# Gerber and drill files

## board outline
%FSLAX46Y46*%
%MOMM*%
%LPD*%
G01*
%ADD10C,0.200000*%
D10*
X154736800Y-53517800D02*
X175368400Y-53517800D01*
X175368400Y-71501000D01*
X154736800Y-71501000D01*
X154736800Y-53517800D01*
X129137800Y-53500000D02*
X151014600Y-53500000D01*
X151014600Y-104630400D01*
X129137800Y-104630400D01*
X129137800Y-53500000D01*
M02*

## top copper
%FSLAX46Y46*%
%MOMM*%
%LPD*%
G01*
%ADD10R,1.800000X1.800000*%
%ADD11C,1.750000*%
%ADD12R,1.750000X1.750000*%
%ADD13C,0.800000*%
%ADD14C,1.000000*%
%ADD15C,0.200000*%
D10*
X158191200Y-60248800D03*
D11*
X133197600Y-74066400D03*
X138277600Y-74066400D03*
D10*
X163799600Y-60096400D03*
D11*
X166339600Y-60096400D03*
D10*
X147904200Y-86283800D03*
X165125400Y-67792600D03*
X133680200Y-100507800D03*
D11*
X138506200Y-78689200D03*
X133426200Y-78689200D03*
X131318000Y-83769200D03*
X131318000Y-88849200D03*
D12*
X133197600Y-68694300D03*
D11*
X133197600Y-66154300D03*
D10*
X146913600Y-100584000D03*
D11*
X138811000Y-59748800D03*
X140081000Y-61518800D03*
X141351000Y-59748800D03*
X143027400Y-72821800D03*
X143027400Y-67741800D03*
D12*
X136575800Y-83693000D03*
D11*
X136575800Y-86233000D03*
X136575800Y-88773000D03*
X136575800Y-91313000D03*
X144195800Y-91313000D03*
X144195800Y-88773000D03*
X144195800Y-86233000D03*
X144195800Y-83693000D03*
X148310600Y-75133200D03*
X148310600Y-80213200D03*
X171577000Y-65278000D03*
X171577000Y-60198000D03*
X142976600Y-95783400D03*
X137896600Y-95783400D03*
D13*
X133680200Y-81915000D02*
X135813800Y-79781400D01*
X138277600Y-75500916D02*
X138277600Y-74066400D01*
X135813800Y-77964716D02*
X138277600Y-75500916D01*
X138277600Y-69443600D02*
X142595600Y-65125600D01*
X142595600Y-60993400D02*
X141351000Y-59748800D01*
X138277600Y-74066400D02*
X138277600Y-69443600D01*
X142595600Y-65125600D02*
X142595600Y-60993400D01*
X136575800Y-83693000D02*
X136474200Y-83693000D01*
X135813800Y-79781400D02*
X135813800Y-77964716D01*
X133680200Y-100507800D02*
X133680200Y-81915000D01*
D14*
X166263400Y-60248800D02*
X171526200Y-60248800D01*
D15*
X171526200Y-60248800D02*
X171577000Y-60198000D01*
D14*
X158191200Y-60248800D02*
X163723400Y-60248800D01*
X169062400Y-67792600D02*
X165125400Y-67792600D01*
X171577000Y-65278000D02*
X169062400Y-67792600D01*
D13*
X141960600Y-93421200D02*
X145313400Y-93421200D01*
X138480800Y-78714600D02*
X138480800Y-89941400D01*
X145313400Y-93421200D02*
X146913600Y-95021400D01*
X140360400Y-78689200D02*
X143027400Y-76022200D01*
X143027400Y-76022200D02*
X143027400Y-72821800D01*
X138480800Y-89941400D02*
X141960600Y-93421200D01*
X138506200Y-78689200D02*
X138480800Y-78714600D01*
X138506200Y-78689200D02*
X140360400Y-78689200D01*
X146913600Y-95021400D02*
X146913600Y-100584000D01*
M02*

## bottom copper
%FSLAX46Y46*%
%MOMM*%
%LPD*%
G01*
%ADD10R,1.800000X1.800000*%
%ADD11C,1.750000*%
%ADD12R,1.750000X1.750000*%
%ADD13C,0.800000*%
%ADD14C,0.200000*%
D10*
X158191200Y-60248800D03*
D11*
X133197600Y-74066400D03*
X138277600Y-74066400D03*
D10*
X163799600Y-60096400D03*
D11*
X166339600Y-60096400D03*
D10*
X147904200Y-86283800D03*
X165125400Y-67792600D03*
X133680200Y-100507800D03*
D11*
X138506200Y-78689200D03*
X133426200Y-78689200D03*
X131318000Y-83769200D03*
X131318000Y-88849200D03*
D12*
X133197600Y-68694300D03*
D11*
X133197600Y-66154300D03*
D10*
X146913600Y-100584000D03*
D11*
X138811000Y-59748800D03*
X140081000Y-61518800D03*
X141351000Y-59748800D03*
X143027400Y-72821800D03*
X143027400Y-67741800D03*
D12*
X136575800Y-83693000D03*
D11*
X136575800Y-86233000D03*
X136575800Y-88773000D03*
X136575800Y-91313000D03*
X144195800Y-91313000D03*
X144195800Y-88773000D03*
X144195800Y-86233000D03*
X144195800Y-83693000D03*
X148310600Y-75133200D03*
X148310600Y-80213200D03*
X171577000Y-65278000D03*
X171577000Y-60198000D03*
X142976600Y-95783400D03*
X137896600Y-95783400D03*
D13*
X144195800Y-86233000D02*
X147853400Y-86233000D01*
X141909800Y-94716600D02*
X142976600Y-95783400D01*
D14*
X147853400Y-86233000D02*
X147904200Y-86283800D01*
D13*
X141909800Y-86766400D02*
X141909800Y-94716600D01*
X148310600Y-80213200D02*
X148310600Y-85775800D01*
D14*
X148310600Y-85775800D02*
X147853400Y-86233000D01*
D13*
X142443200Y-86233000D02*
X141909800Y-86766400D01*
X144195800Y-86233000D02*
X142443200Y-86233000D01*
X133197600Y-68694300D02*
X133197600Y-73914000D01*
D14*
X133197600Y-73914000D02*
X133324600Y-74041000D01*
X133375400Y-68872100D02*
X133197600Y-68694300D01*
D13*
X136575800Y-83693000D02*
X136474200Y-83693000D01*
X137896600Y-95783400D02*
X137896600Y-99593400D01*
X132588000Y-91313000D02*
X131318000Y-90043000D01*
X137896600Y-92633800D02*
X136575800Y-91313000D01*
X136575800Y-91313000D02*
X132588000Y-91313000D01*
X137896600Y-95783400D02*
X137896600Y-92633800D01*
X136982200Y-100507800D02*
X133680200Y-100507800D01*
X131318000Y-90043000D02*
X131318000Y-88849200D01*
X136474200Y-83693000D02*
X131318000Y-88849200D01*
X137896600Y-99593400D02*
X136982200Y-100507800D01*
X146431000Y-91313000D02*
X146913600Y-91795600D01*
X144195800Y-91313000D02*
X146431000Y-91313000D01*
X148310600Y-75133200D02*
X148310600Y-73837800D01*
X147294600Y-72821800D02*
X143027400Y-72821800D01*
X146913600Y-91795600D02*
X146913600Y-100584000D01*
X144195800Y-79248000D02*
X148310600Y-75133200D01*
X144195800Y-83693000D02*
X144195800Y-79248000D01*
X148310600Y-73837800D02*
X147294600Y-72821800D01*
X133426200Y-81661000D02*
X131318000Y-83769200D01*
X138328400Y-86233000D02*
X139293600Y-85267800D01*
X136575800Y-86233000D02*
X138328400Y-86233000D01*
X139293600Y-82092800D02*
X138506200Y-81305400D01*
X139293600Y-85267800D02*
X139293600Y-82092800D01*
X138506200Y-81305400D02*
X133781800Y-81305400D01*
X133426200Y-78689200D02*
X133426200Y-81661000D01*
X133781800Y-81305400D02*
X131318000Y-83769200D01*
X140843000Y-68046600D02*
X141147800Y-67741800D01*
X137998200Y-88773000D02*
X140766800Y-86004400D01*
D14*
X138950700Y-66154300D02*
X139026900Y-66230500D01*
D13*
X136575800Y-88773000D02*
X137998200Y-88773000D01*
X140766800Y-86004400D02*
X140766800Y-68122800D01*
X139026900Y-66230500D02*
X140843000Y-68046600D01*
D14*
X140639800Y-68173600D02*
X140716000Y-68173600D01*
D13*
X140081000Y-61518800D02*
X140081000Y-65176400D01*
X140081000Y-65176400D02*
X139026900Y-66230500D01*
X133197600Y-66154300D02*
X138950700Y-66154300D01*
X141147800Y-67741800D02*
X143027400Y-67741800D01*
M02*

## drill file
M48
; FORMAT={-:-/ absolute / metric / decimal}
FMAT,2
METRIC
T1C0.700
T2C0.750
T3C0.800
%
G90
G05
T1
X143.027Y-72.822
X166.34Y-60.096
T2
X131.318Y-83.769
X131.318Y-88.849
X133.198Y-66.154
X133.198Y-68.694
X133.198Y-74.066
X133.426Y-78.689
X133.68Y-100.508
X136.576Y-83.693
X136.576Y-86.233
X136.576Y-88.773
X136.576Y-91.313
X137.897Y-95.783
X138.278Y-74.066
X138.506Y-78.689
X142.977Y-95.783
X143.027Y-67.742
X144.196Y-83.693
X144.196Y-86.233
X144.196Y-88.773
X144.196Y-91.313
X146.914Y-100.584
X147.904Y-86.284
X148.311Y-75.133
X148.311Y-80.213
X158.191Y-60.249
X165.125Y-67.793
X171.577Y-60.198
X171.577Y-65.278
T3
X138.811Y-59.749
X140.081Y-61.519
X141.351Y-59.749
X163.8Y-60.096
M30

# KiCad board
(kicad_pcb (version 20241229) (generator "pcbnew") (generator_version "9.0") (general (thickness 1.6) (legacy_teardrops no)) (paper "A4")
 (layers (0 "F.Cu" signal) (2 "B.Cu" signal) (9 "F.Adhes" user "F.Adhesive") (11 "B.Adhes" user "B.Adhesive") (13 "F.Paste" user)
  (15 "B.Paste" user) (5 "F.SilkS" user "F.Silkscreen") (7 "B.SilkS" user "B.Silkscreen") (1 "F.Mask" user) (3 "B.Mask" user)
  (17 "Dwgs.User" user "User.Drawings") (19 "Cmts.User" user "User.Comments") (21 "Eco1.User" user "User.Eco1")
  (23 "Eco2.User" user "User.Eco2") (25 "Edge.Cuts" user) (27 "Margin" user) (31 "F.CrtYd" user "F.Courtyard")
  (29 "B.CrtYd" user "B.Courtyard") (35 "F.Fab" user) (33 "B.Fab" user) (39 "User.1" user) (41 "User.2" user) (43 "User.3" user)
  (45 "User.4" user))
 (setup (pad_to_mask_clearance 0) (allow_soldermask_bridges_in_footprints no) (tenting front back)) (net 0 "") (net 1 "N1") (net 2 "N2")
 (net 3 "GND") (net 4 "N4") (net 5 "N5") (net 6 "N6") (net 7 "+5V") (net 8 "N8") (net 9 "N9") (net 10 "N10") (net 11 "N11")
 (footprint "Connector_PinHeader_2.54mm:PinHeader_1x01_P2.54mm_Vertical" (layer "F.Cu") (at 158.1912 60.2488)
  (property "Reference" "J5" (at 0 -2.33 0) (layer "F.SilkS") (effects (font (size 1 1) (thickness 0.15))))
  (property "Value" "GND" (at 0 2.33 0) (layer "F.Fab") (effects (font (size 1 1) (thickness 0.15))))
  (pad "1" thru_hole rect (at 0 0) (size 1.8 1.8) (drill 0.75) (layers "*.Cu" "*.Mask") (remove_unused_layers no) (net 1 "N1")))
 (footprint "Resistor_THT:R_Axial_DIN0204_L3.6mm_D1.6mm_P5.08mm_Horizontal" (layer "F.Cu") (at 133.1976 74.0664)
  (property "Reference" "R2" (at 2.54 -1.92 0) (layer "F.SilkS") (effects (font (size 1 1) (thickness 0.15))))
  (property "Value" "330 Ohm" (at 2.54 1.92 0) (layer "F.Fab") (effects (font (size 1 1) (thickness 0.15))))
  (pad "1" thru_hole circle (at 0 0) (size 1.75 1.75) (drill 0.75) (layers "*.Cu" "*.Mask") (remove_unused_layers no) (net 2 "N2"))
  (pad "2" thru_hole circle (at 5.08 0) (size 1.75 1.75) (drill 0.75) (layers "*.Cu" "*.Mask") (remove_unused_layers no) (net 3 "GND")))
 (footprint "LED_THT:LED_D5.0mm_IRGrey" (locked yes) (layer "F.Cu") (at 163.7996 60.0964)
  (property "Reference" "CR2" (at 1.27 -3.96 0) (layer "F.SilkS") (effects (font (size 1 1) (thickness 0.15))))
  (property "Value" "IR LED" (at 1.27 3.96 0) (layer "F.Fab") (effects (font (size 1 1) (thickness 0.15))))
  (pad "1" thru_hole rect (at 0 0) (size 1.8 1.8) (drill 0.8) (layers "*.Cu" "*.Mask") (remove_unused_layers no) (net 1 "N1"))
  (pad "2" thru_hole circle (at 2.54 0) (size 1.75 1.75) (drill 0.7) (layers "*.Cu" "*.Mask") (remove_unused_layers no) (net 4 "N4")))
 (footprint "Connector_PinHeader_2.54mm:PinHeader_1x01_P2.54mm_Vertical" (layer "F.Cu") (at 147.9042 86.2838)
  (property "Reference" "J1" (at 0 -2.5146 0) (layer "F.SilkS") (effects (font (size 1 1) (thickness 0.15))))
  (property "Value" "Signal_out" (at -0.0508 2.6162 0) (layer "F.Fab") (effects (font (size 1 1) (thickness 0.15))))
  (pad "1" thru_hole rect (at 0 0) (size 1.8 1.8) (drill 0.75) (layers "*.Cu" "*.Mask") (remove_unused_layers no) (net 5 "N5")))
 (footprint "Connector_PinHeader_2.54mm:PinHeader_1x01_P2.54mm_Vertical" (layer "F.Cu") (at 165.1254 67.7926)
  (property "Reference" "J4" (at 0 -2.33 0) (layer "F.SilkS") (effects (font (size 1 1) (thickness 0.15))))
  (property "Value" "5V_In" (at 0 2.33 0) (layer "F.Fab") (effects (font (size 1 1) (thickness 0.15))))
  (pad "1" thru_hole rect (at 0 0) (size 1.8 1.8) (drill 0.75) (layers "*.Cu" "*.Mask") (remove_unused_layers no) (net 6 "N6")))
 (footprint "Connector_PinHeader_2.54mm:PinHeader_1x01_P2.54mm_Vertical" (layer "F.Cu") (at 133.6802 100.5078)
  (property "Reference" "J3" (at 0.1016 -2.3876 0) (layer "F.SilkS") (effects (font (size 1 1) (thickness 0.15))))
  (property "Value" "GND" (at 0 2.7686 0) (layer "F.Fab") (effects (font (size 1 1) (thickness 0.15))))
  (pad "1" thru_hole rect (at 0 0) (size 1.8 1.8) (drill 0.75) (layers "*.Cu" "*.Mask") (remove_unused_layers no) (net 3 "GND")))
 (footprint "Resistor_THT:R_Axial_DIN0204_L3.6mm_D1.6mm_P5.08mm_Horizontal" (layer "F.Cu") (at 138.5062 78.6892 180)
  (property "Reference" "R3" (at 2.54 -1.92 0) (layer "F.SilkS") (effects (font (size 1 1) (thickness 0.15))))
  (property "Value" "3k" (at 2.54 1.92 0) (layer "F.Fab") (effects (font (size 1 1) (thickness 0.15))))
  (pad "1" thru_hole circle (at 0 0 180) (size 1.75 1.75) (drill 0.75) (layers "*.Cu" "*.Mask") (remove_unused_layers no) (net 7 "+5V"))
  (pad "2" thru_hole circle (at 5.08 0 180) (size 1.75 1.75) (drill 0.75) (layers "*.Cu" "*.Mask") (remove_unused_layers no) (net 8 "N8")))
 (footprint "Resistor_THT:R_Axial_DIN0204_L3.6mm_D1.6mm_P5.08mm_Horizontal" (layer "F.Cu") (at 131.318 83.7692 -90)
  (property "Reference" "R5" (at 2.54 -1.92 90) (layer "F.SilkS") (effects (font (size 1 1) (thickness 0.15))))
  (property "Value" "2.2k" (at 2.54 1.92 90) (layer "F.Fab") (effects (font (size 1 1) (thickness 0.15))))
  (pad "1" thru_hole circle (at 0 0 270) (size 1.75 1.75) (drill 0.75) (layers "*.Cu" "*.Mask") (remove_unused_layers no) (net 8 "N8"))
  (pad "2" thru_hole circle (at 5.08 0 270) (size 1.75 1.75) (drill 0.75) (layers "*.Cu" "*.Mask") (remove_unused_layers no) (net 3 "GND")))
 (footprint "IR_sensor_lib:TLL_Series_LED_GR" (layer "F.Cu") (at 133.1976 68.6943 90)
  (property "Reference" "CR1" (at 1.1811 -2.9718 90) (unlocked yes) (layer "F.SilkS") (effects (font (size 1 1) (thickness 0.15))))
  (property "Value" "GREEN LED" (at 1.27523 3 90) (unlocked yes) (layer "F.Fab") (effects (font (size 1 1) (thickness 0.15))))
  (pad "1" thru_hole rect (at 0 0 90) (size 1.75 1.75) (drill 0.75) (layers "*.Cu" "*.Mask") (remove_unused_layers no) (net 2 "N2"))
  (pad "2" thru_hole circle (at 2.54 0 90) (size 1.75 1.75) (drill 0.75) (layers "*.Cu" "*.Mask") (remove_unused_layers no) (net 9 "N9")))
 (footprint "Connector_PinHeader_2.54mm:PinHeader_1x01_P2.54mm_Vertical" (layer "F.Cu") (at 146.9136 100.584)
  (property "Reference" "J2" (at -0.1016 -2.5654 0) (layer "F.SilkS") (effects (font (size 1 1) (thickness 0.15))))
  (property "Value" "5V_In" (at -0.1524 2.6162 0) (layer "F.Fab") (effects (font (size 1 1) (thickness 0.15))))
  (pad "1" thru_hole rect (at 0 0) (size 1.8 1.8) (drill 0.75) (layers "*.Cu" "*.Mask") (remove_unused_layers no) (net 7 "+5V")))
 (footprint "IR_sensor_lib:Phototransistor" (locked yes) (layer "F.Cu") (at 140.081 60.2488 180)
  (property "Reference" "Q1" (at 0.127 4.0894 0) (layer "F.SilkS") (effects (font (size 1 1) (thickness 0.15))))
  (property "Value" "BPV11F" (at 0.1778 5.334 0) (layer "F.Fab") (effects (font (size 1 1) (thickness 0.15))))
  (pad "B" thru_hole circle (at 1.27 0.5 180) (size 1.75 1.75) (drill 0.8) (layers "*.Cu" "*.Mask") (remove_unused_layers no) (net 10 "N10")
   (solder_mask_margin 0.102))
  (pad "C" thru_hole circle (at 0 -1.27 180) (size 1.75 1.75) (drill 0.8) (layers "*.Cu" "*.Mask") (remove_unused_layers no) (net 9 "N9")
   (solder_mask_margin 0.102))
  (pad "E" thru_hole circle (at -1.27 0.5 180) (size 1.75 1.75) (drill 0.8) (layers "*.Cu" "*.Mask") (remove_unused_layers no) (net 3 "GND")
   (solder_mask_margin 0.102)))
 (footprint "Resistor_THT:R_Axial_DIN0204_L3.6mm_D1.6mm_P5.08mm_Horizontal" (layer "F.Cu") (at 143.0274 72.8218 90)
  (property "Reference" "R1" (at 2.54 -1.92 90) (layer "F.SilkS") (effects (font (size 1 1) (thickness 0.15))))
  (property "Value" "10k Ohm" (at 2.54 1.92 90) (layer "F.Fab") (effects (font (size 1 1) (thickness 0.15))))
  (pad "1" thru_hole circle (at 0 0 90) (size 1.75 1.75) (drill 0.7) (layers "*.Cu" "*.Mask") (remove_unused_layers no) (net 7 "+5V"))
  (pad "2" thru_hole circle (at 5.08 0 90) (size 1.75 1.75) (drill 0.75) (layers "*.Cu" "*.Mask") (remove_unused_layers no) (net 9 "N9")))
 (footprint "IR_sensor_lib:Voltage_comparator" (layer "F.Cu") (at 140.6878 88.083)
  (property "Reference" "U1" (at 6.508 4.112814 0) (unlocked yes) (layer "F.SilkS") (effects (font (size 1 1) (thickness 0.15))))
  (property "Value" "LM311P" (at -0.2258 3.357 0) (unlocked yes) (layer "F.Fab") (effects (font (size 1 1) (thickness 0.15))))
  (pad "1" thru_hole rect (at -4.112 -4.39) (size 1.75 1.75) (drill 0.75) (layers "*.Cu" "*.Mask") (remove_unused_layers no) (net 3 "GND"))
  (pad "2" thru_hole circle (at -4.112 -1.85) (size 1.75 1.75) (drill 0.75) (layers "*.Cu" "*.Mask") (remove_unused_layers no) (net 8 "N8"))
  (pad "3" thru_hole circle (at -4.112 0.69) (size 1.75 1.75) (drill 0.75) (layers "*.Cu" "*.Mask") (remove_unused_layers no) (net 9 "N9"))
  (pad "4" thru_hole circle (at -4.112 3.23) (size 1.75 1.75) (drill 0.75) (layers "*.Cu" "*.Mask") (remove_unused_layers no) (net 3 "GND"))
  (pad "5" thru_hole circle (at 3.508 3.23) (size 1.75 1.75) (drill 0.75) (layers "*.Cu" "*.Mask") (remove_unused_layers no) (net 7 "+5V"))
  (pad "6" thru_hole circle (at 3.508 0.69) (size 1.75 1.75) (drill 0.75) (layers "*.Cu" "*.Mask") (remove_unused_layers no) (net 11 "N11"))
  (pad "7" thru_hole circle (at 3.508 -1.85) (size 1.75 1.75) (drill 0.75) (layers "*.Cu" "*.Mask") (remove_unused_layers no) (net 5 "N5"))
  (pad "8" thru_hole circle (at 3.508 -4.39) (size 1.75 1.75) (drill 0.75) (layers "*.Cu" "*.Mask") (remove_unused_layers no) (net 7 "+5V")))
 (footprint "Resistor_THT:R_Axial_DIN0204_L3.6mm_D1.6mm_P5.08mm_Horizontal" (layer "F.Cu") (at 148.3106 75.1332 -90)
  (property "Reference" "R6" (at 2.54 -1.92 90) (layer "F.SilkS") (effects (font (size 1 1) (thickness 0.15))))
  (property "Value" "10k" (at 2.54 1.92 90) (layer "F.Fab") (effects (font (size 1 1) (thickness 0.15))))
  (pad "1" thru_hole circle (at 0 0 270) (size 1.75 1.75) (drill 0.75) (layers "*.Cu" "*.Mask") (remove_unused_layers no) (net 7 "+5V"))
  (pad "2" thru_hole circle (at 5.08 0 270) (size 1.75 1.75) (drill 0.75) (layers "*.Cu" "*.Mask") (remove_unused_layers no) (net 5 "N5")))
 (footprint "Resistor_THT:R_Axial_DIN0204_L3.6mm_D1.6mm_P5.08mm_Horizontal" (layer "F.Cu") (at 171.577 65.278 90)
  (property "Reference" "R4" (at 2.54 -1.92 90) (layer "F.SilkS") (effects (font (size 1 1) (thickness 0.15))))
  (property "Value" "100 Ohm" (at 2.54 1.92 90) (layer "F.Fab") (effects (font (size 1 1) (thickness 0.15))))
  (pad "1" thru_hole circle (at 0 0 90) (size 1.75 1.75) (drill 0.75) (layers "*.Cu" "*.Mask") (remove_unused_layers no) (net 6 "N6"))
  (pad "2" thru_hole circle (at 5.08 0 90) (size 1.75 1.75) (drill 0.75) (layers "*.Cu" "*.Mask") (remove_unused_layers no) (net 4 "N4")))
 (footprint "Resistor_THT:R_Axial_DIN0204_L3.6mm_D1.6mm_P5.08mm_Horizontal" (layer "F.Cu") (at 142.9766 95.7834 180)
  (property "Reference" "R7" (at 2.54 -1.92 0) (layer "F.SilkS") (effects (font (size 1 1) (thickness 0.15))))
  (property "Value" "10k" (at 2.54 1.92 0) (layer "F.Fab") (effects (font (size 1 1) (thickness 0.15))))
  (pad "1" thru_hole circle (at 0 0 180) (size 1.75 1.75) (drill 0.75) (layers "*.Cu" "*.Mask") (remove_unused_layers no) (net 5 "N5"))
  (pad "2" thru_hole circle (at 5.08 0 180) (size 1.75 1.75) (drill 0.75) (layers "*.Cu" "*.Mask") (remove_unused_layers no) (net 3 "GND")))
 (gr_rect (start 154.7368 53.5178) (end 175.3684 71.501) (stroke (width 0.2) (type solid)) (fill no) (layer "Edge.Cuts"))
 (gr_rect (start 129.1378 53.5) (end 151.0146 104.6304) (stroke (width 0.2) (type solid)) (fill no) (layer "Edge.Cuts"))
 (segment (start 144.1958 86.233) (end 147.8534 86.233) (width 0.8) (layer "B.Cu") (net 5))
 (segment (start 141.9098 94.7166) (end 142.9766 95.7834) (width 0.8) (layer "B.Cu") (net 5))
 (segment (start 147.8534 86.233) (end 147.9042 86.2838) (width 0.2) (layer "B.Cu") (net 5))
 (segment (start 141.9098 86.7664) (end 141.9098 94.7166) (width 0.8) (layer "B.Cu") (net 5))
 (segment (start 148.3106 80.2132) (end 148.3106 85.7758) (width 0.8) (layer "B.Cu") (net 5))
 (segment (start 148.3106 85.7758) (end 147.8534 86.233) (width 0.2) (layer "B.Cu") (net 5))
 (segment (start 142.4432 86.233) (end 141.9098 86.7664) (width 0.8) (layer "B.Cu") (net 5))
 (segment (start 144.1958 86.233) (end 142.4432 86.233) (width 0.8) (layer "B.Cu") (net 5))
 (segment (start 133.1976 68.6943) (end 133.1976 73.914) (width 0.8) (layer "B.Cu") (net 2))
 (segment (start 133.1976 73.914) (end 133.3246 74.041) (width 0.2) (layer "B.Cu") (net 2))
 (segment (start 133.3754 68.8721) (end 133.1976 68.6943) (width 0.2) (layer "B.Cu") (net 2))
 (segment (start 133.6802 81.915) (end 135.8138 79.7814) (width 0.8) (layer "F.Cu") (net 3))
 (segment (start 138.2776 75.500916) (end 138.2776 74.0664) (width 0.8) (layer "F.Cu") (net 3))
 (segment (start 135.8138 77.964716) (end 138.2776 75.500916) (width 0.8) (layer "F.Cu") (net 3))
 (segment (start 138.2776 69.4436) (end 142.5956 65.1256) (width 0.8) (layer "F.Cu") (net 3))
 (segment (start 142.5956 60.9934) (end 141.351 59.7488) (width 0.8) (layer "F.Cu") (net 3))
 (segment (start 138.2776 74.0664) (end 138.2776 69.4436) (width 0.8) (layer "F.Cu") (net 3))
 (segment (start 142.5956 65.1256) (end 142.5956 60.9934) (width 0.8) (layer "F.Cu") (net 3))
 (segment (start 136.5758 83.693) (end 136.4742 83.693) (width 0.8) (layer "F.Cu") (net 3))
 (segment (start 135.8138 79.7814) (end 135.8138 77.964716) (width 0.8) (layer "F.Cu") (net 3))
 (segment (start 133.6802 100.5078) (end 133.6802 81.915) (width 0.8) (layer "F.Cu") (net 3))
 (segment (start 136.5758 83.693) (end 136.4742 83.693) (width 0.8) (layer "B.Cu") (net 3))
 (segment (start 137.8966 95.7834) (end 137.8966 99.5934) (width 0.8) (layer "B.Cu") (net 3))
 (segment (start 132.588 91.313) (end 131.318 90.043) (width 0.8) (layer "B.Cu") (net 3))
 (segment (start 137.8966 92.6338) (end 136.5758 91.313) (width 0.8) (layer "B.Cu") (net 3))
 (segment (start 136.5758 91.313) (end 132.588 91.313) (width 0.8) (layer "B.Cu") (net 3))
 (segment (start 137.8966 95.7834) (end 137.8966 92.6338) (width 0.8) (layer "B.Cu") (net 3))
 (segment (start 136.9822 100.5078) (end 133.6802 100.5078) (width 0.8) (layer "B.Cu") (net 3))
 (segment (start 131.318 90.043) (end 131.318 88.8492) (width 0.8) (layer "B.Cu") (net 3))
 (segment (start 136.4742 83.693) (end 131.318 88.8492) (width 0.8) (layer "B.Cu") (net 3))
 (segment (start 137.8966 99.5934) (end 136.9822 100.5078) (width 0.8) (layer "B.Cu") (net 3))
 (segment (start 166.2634 60.2488) (end 171.5262 60.2488) (width 1) (layer "F.Cu") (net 4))
 (segment (start 171.5262 60.2488) (end 171.577 60.198) (width 0.2) (layer "F.Cu") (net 4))
 (segment (start 158.1912 60.2488) (end 163.7234 60.2488) (width 1) (layer "F.Cu") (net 1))
 (segment (start 169.0624 67.7926) (end 165.1254 67.7926) (width 1) (layer "F.Cu") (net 6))
 (segment (start 171.577 65.278) (end 169.0624 67.7926) (width 1) (layer "F.Cu") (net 6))
 (segment (start 141.9606 93.4212) (end 145.3134 93.4212) (width 0.8) (layer "F.Cu") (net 7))
 (segment (start 138.4808 78.7146) (end 138.4808 89.9414) (width 0.8) (layer "F.Cu") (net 7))
 (segment (start 145.3134 93.4212) (end 146.9136 95.0214) (width 0.8) (layer "F.Cu") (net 7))
 (segment (start 140.3604 78.6892) (end 143.0274 76.0222) (width 0.8) (layer "F.Cu") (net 7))
 (segment (start 143.0274 76.0222) (end 143.0274 72.8218) (width 0.8) (layer "F.Cu") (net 7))
 (segment (start 138.4808 89.9414) (end 141.9606 93.4212) (width 0.8) (layer "F.Cu") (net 7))
 (segment (start 138.5062 78.6892) (end 138.4808 78.7146) (width 0.8) (layer "F.Cu") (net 7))
 (segment (start 138.5062 78.6892) (end 140.3604 78.6892) (width 0.8) (layer "F.Cu") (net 7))
 (segment (start 146.9136 95.0214) (end 146.9136 100.584) (width 0.8) (layer "F.Cu") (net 7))
 (segment (start 146.431 91.313) (end 146.9136 91.7956) (width 0.8) (layer "B.Cu") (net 7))
 (segment (start 144.1958 91.313) (end 146.431 91.313) (width 0.8) (layer "B.Cu") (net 7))
 (segment (start 148.3106 75.1332) (end 148.3106 73.8378) (width 0.8) (layer "B.Cu") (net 7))
 (segment (start 147.2946 72.8218) (end 143.0274 72.8218) (width 0.8) (layer "B.Cu") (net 7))
 (segment (start 146.9136 91.7956) (end 146.9136 100.584) (width 0.8) (layer "B.Cu") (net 7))
 (segment (start 144.1958 79.248) (end 148.3106 75.1332) (width 0.8) (layer "B.Cu") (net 7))
 (segment (start 144.1958 83.693) (end 144.1958 79.248) (width 0.8) (layer "B.Cu") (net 7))
 (segment (start 148.3106 73.8378) (end 147.2946 72.8218) (width 0.8) (layer "B.Cu") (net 7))
 (segment (start 133.4262 81.661) (end 131.318 83.7692) (width 0.8) (layer "B.Cu") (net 8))
 (segment (start 138.3284 86.233) (end 139.2936 85.2678) (width 0.8) (layer "B.Cu") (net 8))
 (segment (start 136.5758 86.233) (end 138.3284 86.233) (width 0.8) (layer "B.Cu") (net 8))
 (segment (start 139.2936 82.0928) (end 138.5062 81.3054) (width 0.8) (layer "B.Cu") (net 8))
 (segment (start 139.2936 85.2678) (end 139.2936 82.0928) (width 0.8) (layer "B.Cu") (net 8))
 (segment (start 138.5062 81.3054) (end 133.7818 81.3054) (width 0.8) (layer "B.Cu") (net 8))
 (segment (start 133.4262 78.6892) (end 133.4262 81.661) (width 0.8) (layer "B.Cu") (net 8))
 (segment (start 133.7818 81.3054) (end 131.318 83.7692) (width 0.8) (layer "B.Cu") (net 8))
 (segment (start 140.843 68.0466) (end 141.1478 67.7418) (width 0.8) (layer "B.Cu") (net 9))
 (segment (start 137.9982 88.773) (end 140.7668 86.0044) (width 0.8) (layer "B.Cu") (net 9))
 (segment (start 138.9507 66.1543) (end 139.0269 66.2305) (width 0.2) (layer "B.Cu") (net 9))
 (segment (start 136.5758 88.773) (end 137.9982 88.773) (width 0.8) (layer "B.Cu") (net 9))
 (segment (start 140.7668 86.0044) (end 140.7668 68.1228) (width 0.8) (layer "B.Cu") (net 9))
 (segment (start 139.0269 66.2305) (end 140.843 68.0466) (width 0.8) (layer "B.Cu") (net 9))
 (segment (start 140.6398 68.1736) (end 140.716 68.1736) (width 0.2) (layer "B.Cu") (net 9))
 (segment (start 140.081 61.5188) (end 140.081 65.1764) (width 0.8) (layer "B.Cu") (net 9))
 (segment (start 140.081 65.1764) (end 139.0269 66.2305) (width 0.8) (layer "B.Cu") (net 9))
 (segment (start 133.1976 66.1543) (end 138.9507 66.1543) (width 0.8) (layer "B.Cu") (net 9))
 (segment (start 141.1478 67.7418) (end 143.0274 67.7418) (width 0.8) (layer "B.Cu") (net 9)))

